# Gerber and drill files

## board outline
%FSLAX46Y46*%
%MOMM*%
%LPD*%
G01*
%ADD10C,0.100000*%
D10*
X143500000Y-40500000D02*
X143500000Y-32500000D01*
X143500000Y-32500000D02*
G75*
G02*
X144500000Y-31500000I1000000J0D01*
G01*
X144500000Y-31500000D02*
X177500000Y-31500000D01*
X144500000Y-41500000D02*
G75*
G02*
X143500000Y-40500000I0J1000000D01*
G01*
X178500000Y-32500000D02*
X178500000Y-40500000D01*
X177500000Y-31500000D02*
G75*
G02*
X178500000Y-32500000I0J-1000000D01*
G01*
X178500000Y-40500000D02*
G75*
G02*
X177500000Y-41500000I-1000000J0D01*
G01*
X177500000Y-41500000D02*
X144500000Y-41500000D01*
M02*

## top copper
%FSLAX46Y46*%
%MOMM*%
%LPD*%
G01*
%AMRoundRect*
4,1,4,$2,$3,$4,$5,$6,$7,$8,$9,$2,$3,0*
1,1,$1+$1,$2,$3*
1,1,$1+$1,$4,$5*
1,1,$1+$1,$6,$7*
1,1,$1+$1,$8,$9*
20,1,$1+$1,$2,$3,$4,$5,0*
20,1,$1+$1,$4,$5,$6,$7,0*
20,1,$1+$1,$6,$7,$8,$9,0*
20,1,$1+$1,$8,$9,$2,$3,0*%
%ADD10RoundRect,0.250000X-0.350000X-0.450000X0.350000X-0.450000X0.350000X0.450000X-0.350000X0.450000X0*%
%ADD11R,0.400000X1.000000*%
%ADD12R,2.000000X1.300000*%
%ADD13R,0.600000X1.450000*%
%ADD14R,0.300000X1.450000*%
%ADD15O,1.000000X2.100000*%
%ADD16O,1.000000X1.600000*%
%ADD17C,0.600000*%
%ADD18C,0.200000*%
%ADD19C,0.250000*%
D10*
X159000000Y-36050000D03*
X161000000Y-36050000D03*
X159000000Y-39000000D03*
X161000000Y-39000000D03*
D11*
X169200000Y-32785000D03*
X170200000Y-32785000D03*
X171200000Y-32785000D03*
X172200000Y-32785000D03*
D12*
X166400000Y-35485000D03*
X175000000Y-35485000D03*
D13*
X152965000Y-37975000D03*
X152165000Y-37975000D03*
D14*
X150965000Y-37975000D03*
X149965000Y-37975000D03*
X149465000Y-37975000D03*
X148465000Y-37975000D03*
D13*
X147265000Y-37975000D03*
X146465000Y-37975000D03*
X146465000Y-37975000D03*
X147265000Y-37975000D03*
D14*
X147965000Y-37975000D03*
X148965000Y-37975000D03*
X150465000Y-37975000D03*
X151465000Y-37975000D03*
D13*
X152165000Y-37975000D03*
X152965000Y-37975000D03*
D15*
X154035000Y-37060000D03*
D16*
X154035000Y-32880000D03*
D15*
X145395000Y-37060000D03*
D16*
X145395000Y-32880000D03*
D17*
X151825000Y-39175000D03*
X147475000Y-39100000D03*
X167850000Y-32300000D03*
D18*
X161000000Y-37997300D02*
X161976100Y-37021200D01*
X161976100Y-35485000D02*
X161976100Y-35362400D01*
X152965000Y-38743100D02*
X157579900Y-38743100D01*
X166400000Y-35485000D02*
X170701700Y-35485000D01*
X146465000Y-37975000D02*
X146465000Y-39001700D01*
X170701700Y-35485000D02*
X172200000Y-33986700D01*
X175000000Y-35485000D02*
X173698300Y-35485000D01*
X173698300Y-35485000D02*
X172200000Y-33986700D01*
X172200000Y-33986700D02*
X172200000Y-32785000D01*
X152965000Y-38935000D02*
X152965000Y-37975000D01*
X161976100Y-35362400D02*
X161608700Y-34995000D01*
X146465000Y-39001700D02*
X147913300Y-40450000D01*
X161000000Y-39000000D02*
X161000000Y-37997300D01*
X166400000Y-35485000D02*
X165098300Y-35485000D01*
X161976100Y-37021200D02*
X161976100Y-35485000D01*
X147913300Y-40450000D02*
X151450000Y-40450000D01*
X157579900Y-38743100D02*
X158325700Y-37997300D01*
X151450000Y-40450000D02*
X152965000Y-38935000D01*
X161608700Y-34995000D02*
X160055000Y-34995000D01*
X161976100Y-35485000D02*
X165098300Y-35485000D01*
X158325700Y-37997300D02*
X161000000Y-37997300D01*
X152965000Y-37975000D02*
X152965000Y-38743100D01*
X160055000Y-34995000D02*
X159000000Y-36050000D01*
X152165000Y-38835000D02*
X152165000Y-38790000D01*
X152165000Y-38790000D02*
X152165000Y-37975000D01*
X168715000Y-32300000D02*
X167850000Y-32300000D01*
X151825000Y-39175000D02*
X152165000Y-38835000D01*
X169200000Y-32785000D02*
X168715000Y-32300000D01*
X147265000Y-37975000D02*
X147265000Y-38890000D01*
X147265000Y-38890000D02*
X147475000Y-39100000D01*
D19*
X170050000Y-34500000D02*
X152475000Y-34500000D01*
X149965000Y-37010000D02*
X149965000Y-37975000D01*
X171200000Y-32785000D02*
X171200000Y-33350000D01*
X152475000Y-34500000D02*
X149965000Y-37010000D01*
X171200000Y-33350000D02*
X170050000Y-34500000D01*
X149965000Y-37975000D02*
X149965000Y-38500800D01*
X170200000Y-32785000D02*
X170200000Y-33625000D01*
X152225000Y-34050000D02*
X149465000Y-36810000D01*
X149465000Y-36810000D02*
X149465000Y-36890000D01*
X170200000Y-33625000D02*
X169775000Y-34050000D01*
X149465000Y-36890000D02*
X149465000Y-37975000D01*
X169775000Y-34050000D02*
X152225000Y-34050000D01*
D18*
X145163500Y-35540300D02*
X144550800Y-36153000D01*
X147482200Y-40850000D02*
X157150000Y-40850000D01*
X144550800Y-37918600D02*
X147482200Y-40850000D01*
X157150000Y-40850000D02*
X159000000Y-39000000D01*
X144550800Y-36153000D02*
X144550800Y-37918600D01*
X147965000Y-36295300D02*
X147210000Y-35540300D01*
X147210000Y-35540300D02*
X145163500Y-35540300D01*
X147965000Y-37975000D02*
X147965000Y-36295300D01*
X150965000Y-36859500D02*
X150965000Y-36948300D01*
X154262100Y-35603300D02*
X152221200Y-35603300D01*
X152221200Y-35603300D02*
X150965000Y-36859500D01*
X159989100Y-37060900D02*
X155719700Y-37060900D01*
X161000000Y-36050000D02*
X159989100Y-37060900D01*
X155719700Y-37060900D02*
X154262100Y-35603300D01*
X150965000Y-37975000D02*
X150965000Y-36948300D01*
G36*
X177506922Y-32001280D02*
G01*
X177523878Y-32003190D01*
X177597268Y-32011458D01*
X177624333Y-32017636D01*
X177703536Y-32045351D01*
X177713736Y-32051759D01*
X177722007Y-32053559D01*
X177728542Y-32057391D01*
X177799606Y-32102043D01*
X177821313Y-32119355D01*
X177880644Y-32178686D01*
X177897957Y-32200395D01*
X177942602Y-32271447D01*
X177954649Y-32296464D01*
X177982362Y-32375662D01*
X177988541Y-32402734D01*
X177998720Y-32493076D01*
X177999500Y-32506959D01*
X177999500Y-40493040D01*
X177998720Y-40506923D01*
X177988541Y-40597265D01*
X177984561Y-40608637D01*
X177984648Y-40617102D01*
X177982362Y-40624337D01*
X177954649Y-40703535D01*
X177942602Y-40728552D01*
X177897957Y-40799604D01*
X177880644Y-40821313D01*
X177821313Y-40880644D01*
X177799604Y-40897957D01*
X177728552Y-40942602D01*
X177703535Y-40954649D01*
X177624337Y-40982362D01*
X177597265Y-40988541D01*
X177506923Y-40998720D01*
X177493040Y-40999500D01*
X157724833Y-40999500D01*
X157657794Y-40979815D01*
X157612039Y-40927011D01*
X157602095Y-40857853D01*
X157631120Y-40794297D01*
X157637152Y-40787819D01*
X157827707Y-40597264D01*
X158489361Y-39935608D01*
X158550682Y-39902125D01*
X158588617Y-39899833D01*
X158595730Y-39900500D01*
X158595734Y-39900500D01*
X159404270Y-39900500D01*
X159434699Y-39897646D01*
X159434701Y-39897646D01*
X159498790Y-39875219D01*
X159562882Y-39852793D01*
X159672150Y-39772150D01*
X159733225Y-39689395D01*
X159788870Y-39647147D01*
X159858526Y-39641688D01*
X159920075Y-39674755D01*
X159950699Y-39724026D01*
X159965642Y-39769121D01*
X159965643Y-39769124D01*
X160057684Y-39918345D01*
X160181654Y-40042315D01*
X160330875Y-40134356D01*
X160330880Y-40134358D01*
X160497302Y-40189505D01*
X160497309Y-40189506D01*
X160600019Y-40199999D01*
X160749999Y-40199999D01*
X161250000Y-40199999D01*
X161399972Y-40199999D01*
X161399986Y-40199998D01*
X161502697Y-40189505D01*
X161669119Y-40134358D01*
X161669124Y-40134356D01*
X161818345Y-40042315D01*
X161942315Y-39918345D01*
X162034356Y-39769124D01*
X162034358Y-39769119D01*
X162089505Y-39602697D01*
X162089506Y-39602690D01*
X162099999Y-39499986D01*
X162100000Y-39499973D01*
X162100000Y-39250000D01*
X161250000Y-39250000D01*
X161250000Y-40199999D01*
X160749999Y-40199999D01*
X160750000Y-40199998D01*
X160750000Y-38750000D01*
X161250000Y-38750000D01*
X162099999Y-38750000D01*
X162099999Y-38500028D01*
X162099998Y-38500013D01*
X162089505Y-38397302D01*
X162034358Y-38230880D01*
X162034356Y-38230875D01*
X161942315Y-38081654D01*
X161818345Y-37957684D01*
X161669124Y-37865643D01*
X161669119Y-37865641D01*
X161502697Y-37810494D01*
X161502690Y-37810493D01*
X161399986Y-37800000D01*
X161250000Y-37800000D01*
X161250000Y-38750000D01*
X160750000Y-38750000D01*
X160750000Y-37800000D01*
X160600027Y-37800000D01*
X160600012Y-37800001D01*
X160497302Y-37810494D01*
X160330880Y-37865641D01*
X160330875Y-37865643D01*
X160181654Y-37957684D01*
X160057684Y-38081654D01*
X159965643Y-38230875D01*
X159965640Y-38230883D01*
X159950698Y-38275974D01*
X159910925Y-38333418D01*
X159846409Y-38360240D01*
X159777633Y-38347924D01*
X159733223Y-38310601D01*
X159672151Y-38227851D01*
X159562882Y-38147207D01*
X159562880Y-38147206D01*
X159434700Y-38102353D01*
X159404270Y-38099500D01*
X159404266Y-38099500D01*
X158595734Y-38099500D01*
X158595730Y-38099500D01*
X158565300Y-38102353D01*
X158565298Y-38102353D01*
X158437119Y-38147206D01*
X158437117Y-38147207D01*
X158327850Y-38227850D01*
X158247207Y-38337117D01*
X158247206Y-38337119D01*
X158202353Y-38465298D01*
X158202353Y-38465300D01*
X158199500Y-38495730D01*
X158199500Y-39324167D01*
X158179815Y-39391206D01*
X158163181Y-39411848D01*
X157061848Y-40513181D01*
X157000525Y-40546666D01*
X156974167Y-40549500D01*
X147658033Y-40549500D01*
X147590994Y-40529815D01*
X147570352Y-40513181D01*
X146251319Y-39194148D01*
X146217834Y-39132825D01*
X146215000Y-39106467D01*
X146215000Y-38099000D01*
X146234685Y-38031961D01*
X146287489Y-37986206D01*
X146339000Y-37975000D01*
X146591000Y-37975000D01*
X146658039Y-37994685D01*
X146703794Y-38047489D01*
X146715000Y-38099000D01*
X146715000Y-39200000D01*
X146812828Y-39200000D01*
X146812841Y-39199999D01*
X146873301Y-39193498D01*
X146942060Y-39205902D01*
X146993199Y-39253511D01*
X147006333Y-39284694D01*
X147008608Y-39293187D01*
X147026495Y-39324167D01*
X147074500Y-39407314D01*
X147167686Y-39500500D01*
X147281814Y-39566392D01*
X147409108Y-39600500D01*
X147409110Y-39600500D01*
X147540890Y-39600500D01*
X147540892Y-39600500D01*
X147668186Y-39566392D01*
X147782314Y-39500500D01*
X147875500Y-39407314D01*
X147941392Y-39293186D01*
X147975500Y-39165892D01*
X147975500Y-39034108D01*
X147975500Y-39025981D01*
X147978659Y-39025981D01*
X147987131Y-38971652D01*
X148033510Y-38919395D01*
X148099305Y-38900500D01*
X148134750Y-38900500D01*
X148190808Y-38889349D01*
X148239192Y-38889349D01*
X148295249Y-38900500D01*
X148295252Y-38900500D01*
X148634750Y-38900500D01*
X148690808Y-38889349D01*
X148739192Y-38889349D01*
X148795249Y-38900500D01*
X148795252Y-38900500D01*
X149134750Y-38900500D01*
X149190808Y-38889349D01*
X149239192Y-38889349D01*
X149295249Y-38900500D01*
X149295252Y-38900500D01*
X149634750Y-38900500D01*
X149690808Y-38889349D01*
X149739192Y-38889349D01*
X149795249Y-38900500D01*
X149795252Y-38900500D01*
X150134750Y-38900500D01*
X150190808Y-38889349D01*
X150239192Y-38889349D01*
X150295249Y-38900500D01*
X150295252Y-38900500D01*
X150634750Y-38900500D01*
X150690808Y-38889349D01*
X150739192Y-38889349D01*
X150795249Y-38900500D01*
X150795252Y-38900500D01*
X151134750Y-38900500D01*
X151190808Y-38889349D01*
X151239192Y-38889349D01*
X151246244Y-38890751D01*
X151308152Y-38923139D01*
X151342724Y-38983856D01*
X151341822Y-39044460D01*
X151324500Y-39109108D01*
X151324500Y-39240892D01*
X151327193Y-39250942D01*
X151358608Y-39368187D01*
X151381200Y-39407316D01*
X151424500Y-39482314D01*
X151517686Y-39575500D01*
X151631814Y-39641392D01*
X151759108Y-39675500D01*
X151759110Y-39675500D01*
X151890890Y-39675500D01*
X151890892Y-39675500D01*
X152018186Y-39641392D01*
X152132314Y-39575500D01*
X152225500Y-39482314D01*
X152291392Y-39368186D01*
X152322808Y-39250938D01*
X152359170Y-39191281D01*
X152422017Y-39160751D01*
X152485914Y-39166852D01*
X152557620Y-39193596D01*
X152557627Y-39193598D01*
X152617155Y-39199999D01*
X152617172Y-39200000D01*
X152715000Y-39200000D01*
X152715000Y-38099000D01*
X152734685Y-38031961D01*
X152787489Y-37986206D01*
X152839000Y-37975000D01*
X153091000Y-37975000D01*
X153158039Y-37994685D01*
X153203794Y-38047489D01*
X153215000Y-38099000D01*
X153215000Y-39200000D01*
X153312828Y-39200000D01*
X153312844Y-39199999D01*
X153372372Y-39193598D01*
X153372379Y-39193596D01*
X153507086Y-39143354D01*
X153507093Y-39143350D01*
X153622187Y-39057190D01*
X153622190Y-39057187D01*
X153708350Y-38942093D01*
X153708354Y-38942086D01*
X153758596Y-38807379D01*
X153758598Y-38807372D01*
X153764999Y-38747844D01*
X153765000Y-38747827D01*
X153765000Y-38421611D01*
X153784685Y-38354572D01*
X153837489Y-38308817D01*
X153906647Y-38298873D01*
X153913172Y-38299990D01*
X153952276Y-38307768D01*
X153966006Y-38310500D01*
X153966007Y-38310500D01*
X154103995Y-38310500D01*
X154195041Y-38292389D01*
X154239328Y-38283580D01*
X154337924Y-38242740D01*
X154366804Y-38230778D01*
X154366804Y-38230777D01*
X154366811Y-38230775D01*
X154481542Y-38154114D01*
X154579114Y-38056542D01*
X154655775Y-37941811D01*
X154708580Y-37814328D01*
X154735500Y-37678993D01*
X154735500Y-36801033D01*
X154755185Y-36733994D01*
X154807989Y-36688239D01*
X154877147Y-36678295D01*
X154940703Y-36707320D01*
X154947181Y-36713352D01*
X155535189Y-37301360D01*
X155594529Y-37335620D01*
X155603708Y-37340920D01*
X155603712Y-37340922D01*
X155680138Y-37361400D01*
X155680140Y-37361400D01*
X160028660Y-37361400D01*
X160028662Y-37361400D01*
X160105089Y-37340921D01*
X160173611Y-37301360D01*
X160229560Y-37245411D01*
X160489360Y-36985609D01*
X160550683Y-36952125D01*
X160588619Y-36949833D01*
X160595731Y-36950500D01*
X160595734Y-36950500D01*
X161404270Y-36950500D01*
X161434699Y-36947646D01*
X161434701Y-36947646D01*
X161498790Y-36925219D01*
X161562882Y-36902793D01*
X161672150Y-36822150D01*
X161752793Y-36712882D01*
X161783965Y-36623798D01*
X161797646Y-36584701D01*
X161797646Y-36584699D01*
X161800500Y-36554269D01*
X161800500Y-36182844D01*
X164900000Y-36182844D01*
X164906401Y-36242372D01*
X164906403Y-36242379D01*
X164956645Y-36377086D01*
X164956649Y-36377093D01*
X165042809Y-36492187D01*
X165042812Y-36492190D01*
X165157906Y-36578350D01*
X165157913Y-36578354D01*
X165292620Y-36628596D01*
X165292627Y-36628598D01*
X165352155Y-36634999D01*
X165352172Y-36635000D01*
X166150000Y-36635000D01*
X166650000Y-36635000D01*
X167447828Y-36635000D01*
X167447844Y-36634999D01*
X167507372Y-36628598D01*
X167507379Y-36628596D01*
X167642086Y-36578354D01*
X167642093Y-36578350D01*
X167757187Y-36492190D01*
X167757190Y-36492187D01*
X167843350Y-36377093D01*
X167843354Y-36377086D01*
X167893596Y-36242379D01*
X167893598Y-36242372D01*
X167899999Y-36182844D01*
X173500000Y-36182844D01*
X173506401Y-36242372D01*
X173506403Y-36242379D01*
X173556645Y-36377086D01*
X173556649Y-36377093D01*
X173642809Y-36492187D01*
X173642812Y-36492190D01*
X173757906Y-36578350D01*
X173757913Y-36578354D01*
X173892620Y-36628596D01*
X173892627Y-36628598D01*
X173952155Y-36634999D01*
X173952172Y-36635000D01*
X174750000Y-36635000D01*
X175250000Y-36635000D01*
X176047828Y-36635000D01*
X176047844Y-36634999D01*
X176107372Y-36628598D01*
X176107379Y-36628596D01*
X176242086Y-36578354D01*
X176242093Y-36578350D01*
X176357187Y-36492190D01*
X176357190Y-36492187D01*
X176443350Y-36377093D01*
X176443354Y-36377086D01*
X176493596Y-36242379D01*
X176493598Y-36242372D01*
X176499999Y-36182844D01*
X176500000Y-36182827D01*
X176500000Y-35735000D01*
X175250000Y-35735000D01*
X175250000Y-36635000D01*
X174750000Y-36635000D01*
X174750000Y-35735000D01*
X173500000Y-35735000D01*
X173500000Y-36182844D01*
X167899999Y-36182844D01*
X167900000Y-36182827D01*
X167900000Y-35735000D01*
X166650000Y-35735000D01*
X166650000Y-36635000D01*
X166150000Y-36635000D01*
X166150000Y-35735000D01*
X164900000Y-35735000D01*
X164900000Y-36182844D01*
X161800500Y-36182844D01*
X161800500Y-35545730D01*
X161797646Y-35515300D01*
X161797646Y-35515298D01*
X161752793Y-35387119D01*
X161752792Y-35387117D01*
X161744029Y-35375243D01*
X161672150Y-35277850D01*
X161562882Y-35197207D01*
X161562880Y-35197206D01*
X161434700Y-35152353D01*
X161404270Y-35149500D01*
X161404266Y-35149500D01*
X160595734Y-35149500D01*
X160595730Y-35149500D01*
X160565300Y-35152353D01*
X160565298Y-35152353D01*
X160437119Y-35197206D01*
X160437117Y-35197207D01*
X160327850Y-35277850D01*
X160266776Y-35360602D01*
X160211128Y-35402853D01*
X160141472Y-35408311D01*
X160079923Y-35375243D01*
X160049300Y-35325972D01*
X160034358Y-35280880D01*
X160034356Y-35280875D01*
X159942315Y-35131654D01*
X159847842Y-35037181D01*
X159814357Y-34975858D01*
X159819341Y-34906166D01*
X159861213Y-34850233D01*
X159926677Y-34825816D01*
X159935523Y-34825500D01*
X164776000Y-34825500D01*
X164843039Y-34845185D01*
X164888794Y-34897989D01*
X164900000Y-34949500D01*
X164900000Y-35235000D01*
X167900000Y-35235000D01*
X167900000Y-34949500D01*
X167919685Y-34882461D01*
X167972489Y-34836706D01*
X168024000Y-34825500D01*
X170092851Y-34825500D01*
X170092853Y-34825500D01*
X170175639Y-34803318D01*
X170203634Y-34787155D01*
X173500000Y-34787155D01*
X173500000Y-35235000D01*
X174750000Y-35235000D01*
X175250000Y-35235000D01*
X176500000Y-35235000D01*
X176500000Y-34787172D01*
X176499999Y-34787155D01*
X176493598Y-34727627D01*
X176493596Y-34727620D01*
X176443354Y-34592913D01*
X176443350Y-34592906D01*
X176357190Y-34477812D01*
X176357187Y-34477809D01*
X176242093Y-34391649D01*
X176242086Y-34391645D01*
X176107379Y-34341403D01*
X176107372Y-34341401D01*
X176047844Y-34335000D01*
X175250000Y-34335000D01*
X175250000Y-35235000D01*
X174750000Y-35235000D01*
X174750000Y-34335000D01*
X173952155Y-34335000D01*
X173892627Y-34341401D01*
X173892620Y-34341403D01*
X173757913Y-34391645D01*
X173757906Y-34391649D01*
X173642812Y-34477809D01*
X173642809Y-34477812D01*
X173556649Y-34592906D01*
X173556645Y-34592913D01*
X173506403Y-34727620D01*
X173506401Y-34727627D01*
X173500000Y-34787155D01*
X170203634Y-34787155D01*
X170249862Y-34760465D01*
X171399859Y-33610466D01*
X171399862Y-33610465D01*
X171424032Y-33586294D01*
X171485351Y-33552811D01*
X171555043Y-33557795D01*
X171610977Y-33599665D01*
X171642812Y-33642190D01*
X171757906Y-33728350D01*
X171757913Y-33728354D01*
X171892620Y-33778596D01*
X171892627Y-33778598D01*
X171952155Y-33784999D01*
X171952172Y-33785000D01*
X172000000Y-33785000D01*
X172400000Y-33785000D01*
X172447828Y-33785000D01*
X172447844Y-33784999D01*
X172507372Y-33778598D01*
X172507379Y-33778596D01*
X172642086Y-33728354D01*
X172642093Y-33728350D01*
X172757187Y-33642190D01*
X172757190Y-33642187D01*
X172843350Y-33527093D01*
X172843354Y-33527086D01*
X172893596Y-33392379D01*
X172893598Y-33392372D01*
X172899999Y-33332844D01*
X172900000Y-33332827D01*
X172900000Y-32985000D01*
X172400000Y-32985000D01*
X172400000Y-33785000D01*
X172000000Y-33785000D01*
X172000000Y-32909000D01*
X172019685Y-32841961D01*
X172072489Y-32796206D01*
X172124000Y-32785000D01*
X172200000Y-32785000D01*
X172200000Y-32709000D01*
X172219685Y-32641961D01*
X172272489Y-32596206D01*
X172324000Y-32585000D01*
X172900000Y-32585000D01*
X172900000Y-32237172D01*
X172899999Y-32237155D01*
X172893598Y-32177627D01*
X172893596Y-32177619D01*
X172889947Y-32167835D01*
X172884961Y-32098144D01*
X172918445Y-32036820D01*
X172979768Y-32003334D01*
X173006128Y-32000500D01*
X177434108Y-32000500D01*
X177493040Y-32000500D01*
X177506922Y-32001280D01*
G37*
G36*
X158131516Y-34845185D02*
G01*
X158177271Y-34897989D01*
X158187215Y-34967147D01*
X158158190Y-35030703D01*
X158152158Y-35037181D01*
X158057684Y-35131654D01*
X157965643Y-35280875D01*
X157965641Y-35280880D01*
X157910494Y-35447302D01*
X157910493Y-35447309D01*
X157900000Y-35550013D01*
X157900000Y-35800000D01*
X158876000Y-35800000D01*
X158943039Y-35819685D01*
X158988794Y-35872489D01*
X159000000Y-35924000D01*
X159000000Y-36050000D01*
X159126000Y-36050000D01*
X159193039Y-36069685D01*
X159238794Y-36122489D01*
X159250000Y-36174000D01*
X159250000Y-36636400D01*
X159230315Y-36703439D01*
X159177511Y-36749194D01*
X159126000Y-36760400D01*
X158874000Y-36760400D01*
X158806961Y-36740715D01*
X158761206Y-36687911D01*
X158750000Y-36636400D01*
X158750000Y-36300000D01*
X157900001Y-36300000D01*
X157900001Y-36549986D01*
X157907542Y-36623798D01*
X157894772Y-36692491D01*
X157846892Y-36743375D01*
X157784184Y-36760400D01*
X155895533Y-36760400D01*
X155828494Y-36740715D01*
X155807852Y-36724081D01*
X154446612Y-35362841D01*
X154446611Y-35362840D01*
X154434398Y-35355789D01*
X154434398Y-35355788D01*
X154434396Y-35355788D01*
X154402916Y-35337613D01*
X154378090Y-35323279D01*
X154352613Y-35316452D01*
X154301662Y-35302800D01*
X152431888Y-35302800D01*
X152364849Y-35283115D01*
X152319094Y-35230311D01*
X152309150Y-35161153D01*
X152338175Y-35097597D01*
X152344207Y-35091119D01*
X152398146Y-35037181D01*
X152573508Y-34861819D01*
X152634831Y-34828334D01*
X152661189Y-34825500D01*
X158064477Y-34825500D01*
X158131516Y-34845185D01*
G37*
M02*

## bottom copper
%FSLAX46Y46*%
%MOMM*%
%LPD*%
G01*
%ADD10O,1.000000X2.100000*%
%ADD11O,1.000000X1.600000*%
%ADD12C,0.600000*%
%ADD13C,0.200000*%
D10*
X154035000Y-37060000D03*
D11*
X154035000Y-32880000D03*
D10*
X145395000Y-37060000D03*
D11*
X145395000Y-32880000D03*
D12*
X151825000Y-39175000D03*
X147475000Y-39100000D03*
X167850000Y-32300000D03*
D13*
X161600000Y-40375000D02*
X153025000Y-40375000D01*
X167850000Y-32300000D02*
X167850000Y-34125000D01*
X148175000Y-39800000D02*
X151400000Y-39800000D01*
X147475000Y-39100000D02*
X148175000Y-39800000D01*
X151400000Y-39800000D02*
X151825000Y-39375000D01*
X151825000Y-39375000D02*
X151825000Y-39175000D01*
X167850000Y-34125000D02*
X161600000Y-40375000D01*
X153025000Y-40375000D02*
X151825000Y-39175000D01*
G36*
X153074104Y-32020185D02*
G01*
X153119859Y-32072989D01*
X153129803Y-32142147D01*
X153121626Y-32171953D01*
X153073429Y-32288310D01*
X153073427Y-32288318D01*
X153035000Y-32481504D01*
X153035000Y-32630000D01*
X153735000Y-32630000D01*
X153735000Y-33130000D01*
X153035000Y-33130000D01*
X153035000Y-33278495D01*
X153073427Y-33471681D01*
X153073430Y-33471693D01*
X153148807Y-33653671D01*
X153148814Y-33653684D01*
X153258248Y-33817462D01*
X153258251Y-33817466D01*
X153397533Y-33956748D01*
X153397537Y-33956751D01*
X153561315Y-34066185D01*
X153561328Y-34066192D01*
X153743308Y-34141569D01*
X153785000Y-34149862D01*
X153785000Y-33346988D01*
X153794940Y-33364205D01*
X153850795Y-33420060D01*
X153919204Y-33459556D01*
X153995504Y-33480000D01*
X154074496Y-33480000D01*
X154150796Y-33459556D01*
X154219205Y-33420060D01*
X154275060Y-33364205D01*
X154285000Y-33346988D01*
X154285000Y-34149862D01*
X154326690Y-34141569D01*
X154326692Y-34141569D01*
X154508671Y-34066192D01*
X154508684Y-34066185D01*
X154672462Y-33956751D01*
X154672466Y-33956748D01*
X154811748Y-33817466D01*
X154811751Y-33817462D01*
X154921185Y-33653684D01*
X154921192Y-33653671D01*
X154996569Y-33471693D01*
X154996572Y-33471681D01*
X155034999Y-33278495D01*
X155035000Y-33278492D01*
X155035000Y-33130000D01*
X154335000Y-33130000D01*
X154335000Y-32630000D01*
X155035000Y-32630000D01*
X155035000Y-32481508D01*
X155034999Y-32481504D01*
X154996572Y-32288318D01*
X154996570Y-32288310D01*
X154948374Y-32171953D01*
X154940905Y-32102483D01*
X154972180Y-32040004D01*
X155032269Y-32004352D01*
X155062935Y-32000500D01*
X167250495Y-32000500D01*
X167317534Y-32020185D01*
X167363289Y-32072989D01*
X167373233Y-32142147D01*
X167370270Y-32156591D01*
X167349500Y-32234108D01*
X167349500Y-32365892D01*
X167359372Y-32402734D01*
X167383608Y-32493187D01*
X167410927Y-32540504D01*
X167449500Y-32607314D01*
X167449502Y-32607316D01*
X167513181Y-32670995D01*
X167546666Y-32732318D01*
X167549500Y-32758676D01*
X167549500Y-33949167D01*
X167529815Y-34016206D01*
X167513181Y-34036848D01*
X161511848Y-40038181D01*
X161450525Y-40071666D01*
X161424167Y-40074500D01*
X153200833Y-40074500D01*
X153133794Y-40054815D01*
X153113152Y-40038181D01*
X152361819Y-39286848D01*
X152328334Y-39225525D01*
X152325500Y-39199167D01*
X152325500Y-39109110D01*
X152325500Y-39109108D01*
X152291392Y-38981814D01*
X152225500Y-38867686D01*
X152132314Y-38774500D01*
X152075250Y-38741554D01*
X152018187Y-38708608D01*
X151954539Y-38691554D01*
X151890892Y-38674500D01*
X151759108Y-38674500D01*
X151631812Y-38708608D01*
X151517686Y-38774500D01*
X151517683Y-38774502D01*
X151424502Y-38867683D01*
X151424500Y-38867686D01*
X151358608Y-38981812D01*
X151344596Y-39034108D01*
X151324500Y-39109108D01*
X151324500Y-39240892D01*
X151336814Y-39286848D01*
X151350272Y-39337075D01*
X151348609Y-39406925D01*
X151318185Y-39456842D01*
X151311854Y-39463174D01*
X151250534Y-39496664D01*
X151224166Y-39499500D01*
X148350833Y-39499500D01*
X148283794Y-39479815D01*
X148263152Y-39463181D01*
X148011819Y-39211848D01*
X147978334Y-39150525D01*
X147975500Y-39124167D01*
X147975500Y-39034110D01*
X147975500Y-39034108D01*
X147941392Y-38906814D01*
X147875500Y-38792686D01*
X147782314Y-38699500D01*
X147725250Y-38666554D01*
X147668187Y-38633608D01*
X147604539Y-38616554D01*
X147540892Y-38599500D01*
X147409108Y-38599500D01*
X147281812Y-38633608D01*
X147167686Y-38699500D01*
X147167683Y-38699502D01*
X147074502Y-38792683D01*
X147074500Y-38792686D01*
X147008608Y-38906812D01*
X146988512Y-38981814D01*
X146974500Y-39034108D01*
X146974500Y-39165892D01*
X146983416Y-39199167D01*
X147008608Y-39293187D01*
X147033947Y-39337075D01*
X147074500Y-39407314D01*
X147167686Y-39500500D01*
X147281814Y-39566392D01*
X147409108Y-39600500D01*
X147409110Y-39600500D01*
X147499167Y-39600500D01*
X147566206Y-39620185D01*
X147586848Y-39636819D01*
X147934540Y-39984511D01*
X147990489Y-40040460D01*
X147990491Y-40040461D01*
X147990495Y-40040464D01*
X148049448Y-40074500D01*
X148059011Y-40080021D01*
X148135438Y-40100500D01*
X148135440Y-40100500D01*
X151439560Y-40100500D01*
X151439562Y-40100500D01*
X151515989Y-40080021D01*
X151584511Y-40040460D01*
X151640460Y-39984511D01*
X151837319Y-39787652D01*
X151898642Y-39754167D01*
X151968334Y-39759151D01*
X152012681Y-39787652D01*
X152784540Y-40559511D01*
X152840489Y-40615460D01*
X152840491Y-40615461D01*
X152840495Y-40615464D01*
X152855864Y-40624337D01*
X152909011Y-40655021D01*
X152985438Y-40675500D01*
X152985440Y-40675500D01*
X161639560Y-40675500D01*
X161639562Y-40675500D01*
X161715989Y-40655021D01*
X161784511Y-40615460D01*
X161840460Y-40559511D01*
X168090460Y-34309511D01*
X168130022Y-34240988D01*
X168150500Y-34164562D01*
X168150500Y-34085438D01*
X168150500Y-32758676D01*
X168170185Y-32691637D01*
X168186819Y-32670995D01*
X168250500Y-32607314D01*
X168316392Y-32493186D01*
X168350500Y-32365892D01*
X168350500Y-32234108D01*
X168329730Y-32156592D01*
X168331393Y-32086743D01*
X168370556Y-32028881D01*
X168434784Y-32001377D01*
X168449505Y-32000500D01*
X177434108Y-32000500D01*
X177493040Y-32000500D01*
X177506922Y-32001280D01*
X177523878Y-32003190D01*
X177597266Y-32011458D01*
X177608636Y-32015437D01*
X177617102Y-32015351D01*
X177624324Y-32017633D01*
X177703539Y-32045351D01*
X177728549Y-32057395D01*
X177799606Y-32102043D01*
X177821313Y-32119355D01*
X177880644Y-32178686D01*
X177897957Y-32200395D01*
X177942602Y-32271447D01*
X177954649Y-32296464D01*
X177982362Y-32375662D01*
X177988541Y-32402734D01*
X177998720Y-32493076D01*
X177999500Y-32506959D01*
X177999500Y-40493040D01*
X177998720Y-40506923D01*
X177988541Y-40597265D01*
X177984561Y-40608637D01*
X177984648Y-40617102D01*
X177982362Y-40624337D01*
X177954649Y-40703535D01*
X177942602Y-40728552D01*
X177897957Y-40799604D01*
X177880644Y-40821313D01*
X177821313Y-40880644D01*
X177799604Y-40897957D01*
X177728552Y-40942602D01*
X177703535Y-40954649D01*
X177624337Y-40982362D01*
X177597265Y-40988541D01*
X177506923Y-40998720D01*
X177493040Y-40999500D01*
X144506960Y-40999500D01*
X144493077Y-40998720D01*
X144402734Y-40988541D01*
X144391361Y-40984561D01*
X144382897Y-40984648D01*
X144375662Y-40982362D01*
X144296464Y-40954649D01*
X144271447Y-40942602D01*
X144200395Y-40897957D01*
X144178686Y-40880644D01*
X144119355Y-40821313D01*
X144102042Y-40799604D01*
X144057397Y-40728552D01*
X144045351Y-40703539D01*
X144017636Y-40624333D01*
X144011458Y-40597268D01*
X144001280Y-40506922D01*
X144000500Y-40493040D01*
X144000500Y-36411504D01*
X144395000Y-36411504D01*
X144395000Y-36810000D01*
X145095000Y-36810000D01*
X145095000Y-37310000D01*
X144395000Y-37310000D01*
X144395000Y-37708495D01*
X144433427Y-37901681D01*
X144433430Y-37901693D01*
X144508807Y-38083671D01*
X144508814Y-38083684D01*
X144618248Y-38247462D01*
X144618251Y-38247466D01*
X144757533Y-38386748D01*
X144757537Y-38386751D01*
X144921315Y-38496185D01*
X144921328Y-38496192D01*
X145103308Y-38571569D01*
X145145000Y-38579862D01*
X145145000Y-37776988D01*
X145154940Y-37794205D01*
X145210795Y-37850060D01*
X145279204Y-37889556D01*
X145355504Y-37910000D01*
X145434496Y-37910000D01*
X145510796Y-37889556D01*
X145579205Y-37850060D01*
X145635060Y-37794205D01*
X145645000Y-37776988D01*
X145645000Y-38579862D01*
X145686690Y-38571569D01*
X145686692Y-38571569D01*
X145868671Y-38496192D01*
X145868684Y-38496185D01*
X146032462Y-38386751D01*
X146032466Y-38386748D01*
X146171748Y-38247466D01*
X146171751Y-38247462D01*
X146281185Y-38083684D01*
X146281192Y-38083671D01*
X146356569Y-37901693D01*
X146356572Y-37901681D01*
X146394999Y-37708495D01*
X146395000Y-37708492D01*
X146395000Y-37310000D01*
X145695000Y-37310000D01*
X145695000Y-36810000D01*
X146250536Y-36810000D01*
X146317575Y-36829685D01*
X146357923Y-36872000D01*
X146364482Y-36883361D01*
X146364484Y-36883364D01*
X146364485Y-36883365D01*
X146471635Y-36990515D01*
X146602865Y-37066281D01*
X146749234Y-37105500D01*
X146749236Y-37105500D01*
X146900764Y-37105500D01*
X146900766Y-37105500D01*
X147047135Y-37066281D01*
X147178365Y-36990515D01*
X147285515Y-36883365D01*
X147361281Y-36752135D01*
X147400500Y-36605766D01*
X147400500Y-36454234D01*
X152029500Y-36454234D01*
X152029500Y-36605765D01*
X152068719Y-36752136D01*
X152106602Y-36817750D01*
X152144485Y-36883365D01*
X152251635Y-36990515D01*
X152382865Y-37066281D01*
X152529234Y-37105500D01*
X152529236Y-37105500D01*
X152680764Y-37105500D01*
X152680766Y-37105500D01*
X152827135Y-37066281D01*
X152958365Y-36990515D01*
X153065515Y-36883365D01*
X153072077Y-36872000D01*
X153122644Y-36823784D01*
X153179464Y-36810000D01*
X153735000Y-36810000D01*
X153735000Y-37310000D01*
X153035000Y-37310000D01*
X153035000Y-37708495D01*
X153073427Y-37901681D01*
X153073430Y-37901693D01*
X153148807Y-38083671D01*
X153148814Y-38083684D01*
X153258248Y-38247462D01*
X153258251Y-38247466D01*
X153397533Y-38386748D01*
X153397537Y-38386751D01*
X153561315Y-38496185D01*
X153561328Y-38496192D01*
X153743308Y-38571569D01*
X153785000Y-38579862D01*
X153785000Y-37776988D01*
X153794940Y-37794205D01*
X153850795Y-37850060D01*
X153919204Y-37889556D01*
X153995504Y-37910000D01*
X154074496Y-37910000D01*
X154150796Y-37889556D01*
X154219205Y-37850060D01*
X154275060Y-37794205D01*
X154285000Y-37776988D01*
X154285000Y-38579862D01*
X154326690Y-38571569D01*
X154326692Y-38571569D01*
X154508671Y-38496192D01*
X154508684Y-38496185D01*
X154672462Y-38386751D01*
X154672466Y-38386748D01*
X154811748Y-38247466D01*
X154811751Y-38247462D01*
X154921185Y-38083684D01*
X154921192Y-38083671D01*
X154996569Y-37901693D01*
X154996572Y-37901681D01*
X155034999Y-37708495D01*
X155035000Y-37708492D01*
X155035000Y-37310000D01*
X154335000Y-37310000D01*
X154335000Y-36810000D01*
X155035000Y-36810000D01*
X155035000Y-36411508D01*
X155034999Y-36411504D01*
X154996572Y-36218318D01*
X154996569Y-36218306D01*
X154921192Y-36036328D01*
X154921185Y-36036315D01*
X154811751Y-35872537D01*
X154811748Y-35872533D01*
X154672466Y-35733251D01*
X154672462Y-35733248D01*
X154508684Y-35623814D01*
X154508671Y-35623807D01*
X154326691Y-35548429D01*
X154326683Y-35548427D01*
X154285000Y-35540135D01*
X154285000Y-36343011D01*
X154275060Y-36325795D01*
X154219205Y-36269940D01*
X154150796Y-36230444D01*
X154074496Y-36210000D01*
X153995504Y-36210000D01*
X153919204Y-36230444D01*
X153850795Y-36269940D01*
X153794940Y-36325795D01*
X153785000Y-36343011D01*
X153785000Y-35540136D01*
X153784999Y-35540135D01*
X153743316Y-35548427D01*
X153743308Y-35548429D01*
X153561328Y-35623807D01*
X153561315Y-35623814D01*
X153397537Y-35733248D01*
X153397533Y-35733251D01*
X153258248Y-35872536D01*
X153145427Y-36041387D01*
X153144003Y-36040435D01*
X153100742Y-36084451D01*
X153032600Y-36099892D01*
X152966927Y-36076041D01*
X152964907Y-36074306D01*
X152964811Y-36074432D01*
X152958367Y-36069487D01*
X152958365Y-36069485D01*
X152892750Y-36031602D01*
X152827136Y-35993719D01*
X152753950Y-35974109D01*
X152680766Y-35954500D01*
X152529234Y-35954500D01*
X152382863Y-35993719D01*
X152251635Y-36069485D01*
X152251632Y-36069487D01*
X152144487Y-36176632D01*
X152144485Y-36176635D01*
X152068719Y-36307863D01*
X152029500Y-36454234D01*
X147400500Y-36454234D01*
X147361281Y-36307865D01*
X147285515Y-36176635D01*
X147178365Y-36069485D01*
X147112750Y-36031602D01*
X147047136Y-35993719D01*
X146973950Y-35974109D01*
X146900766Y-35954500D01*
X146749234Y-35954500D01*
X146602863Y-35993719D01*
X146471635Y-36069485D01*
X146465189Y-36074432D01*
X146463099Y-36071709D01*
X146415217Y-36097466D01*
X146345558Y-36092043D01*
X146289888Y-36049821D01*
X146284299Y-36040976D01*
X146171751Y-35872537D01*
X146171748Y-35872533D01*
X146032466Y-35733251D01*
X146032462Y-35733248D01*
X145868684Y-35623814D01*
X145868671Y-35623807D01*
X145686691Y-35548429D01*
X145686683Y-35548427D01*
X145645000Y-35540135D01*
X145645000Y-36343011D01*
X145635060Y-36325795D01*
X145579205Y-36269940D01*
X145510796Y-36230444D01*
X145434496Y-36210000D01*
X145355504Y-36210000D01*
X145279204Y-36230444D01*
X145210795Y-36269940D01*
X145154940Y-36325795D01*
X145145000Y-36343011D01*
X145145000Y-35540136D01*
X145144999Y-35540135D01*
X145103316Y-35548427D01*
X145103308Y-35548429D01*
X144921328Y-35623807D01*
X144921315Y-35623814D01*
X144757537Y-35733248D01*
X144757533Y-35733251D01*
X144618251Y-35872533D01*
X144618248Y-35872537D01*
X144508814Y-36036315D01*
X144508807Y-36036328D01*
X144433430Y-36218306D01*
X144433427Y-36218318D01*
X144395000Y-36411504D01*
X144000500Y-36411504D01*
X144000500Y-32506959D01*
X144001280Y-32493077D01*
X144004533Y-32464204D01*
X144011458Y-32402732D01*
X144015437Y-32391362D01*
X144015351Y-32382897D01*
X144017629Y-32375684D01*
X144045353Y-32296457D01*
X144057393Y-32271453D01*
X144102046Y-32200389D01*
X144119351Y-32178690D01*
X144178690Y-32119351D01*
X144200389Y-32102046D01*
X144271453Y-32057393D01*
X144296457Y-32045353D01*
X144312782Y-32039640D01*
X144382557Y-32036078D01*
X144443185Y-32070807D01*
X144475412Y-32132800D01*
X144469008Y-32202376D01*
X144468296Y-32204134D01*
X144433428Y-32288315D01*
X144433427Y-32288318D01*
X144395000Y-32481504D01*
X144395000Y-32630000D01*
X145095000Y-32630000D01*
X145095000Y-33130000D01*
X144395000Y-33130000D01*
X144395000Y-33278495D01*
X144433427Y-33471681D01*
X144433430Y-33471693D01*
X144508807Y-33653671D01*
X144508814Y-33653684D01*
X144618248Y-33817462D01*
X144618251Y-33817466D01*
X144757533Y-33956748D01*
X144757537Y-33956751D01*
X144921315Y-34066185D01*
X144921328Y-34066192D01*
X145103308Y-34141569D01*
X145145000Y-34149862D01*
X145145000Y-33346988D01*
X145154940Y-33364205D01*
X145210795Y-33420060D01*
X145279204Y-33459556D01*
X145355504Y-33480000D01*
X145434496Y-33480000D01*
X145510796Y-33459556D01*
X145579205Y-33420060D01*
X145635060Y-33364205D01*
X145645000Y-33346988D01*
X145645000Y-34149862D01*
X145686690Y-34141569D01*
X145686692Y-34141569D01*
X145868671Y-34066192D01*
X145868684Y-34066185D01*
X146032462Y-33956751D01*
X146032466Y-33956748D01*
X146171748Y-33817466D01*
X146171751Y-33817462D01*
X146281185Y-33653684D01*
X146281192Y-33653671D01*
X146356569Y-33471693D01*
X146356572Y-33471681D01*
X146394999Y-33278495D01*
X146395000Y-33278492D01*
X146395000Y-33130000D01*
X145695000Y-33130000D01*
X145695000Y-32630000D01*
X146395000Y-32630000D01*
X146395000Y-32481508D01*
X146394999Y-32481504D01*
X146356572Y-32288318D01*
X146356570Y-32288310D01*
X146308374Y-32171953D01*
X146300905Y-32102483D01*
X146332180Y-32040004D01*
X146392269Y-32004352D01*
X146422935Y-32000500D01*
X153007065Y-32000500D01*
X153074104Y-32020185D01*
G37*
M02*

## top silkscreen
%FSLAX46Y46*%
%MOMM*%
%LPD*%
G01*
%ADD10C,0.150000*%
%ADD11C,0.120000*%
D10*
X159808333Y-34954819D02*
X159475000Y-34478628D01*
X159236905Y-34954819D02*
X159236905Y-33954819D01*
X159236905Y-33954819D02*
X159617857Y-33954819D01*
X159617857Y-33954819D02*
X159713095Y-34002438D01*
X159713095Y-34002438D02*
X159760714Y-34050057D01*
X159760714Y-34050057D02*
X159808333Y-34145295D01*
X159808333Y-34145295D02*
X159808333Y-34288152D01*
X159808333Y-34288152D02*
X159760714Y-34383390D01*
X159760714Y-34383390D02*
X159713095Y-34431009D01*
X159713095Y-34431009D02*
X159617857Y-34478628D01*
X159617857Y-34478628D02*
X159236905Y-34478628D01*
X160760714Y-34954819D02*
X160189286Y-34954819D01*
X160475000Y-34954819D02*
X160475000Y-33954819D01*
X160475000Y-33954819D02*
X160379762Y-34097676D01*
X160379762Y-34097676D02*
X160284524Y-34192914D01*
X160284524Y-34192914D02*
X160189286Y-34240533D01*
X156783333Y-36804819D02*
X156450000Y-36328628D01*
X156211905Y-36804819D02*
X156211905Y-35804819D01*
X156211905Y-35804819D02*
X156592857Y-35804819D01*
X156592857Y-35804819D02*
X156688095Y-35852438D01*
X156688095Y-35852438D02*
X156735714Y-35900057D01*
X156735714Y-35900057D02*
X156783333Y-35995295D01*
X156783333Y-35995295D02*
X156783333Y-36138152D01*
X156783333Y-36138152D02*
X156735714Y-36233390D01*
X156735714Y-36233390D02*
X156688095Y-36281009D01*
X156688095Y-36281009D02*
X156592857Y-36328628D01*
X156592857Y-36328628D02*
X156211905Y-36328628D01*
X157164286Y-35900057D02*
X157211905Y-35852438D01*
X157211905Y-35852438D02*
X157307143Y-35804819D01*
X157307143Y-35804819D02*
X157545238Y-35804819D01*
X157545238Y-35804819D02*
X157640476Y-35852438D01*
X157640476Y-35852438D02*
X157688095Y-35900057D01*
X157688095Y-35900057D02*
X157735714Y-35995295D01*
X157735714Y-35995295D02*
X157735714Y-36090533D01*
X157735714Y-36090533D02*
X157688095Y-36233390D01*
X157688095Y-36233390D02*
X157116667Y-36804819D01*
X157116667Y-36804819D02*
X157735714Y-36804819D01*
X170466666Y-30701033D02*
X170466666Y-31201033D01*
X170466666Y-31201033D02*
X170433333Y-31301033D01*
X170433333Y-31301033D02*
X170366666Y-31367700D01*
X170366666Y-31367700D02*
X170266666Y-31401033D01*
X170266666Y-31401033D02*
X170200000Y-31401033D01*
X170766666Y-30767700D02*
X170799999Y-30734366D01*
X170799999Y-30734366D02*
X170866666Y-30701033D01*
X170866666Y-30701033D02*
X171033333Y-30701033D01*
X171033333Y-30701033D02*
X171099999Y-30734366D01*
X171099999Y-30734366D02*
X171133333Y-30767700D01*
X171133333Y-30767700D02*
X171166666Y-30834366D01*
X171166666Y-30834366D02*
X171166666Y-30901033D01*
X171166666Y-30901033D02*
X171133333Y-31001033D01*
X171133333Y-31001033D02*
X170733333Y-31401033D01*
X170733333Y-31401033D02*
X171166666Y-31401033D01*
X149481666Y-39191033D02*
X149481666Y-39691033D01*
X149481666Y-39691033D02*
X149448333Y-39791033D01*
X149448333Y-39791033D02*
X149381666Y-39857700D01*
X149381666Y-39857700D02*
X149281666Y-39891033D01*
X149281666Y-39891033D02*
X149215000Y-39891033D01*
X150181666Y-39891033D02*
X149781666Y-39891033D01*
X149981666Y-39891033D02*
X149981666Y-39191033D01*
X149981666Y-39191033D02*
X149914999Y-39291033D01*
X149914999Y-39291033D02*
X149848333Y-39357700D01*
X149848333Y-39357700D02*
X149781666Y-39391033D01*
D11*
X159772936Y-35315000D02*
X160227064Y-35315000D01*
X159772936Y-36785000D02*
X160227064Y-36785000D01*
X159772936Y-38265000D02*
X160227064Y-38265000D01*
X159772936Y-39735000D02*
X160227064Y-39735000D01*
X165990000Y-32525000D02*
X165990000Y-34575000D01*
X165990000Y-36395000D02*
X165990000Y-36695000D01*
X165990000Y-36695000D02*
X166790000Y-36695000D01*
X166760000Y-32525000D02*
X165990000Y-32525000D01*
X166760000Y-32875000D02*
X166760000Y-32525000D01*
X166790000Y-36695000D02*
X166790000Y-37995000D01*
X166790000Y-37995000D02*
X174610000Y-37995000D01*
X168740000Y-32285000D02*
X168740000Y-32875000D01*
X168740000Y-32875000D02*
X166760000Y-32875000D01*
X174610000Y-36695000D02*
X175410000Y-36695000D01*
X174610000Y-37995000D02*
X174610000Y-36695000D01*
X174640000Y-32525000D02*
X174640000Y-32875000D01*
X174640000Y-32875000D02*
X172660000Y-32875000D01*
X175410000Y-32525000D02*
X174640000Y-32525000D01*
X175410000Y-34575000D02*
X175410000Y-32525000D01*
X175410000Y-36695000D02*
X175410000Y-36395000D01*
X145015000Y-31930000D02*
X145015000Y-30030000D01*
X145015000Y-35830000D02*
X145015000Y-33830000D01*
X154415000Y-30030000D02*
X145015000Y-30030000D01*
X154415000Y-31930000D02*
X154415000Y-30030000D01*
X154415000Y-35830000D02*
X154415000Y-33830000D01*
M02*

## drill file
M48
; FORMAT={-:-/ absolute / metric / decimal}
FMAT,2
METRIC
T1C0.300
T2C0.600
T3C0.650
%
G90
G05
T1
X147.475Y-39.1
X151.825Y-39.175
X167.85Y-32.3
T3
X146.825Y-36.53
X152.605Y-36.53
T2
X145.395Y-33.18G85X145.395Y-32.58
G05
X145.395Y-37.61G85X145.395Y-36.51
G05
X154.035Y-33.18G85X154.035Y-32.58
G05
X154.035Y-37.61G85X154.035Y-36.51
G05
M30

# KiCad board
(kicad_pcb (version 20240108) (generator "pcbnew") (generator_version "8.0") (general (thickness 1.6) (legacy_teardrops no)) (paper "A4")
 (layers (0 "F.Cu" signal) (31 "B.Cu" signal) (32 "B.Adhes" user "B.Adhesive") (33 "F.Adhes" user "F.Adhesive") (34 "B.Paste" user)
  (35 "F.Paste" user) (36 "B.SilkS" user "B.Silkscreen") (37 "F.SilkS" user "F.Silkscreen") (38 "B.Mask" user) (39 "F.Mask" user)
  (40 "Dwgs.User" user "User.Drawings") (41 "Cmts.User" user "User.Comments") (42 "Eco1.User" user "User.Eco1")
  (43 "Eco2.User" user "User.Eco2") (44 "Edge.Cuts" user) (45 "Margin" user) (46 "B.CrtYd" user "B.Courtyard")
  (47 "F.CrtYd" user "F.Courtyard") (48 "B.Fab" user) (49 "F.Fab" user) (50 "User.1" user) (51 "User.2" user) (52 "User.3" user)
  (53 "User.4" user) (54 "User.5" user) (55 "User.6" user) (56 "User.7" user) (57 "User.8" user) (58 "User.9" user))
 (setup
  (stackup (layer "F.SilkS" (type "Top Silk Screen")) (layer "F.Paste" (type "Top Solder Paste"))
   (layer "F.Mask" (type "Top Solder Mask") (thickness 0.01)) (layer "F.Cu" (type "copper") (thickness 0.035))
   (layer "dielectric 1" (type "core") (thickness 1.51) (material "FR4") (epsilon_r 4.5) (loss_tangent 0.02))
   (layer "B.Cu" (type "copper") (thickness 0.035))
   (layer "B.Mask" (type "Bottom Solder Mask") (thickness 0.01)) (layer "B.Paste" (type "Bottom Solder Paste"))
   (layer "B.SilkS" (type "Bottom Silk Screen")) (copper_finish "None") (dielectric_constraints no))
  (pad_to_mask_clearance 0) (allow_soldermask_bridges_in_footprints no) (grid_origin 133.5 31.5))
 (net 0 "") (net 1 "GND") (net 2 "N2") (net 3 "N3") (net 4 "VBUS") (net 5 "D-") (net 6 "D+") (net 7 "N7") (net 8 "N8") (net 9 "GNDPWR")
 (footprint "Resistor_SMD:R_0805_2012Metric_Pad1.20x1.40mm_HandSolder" (layer "F.Cu") (at 160 36.05)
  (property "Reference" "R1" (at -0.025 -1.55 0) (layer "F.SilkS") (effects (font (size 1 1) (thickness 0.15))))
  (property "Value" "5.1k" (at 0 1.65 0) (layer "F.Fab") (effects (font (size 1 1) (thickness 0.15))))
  (fp_line (start -0.227064 -0.735) (end 0.227064 -0.735) (stroke (width 0.12) (type solid)) (layer "F.SilkS"))
  (fp_line (start -0.227064 0.735) (end 0.227064 0.735) (stroke (width 0.12) (type solid)) (layer "F.SilkS"))
  (pad "1" smd roundrect (at -1 0) (size 1.2 1.4) (layers "F.Cu" "F.Paste" "F.Mask") (roundrect_rratio 0.208333) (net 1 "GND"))
  (pad "2" smd roundrect (at 1 0) (size 1.2 1.4) (layers "F.Cu" "F.Paste" "F.Mask") (roundrect_rratio 0.208333) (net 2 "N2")))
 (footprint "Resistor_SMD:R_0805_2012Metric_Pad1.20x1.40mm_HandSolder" (layer "F.Cu") (at 160 39)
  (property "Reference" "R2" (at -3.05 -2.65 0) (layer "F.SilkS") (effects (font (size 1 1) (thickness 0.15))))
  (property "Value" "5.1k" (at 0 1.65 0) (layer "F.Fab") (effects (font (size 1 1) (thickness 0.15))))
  (fp_line (start -0.227064 -0.735) (end 0.227064 -0.735) (stroke (width 0.12) (type solid)) (layer "F.SilkS"))
  (fp_line (start -0.227064 0.735) (end 0.227064 0.735) (stroke (width 0.12) (type solid)) (layer "F.SilkS"))
  (pad "1" smd roundrect (at -1 0) (size 1.2 1.4) (layers "F.Cu" "F.Paste" "F.Mask") (roundrect_rratio 0.208333) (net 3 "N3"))
  (pad "2" smd roundrect (at 1 0) (size 1.2 1.4) (layers "F.Cu" "F.Paste" "F.Mask") (roundrect_rratio 0.208333) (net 1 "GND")))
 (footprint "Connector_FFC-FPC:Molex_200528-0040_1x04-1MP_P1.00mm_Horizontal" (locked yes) (layer "F.Cu") (at 170.7 33.695)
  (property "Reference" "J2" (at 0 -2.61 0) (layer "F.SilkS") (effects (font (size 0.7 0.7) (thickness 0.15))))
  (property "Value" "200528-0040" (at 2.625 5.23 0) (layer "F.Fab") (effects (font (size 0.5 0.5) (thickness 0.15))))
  (fp_line (start -4.71 -1.17) (end -4.71 0.88) (stroke (width 0.12) (type solid)) (layer "F.SilkS"))
  (fp_line (start -4.71 2.7) (end -4.71 3) (stroke (width 0.12) (type solid)) (layer "F.SilkS"))
  (fp_line (start -4.71 3) (end -3.91 3) (stroke (width 0.12) (type solid)) (layer "F.SilkS"))
  (fp_line (start -3.94 -1.17) (end -4.71 -1.17) (stroke (width 0.12) (type solid)) (layer "F.SilkS"))
  (fp_line (start -3.94 -0.82) (end -3.94 -1.17) (stroke (width 0.12) (type solid)) (layer "F.SilkS"))
  (fp_line (start -3.91 3) (end -3.91 4.3) (stroke (width 0.12) (type solid)) (layer "F.SilkS"))
  (fp_line (start -3.91 4.3) (end 3.91 4.3) (stroke (width 0.12) (type solid)) (layer "F.SilkS"))
  (fp_line (start -1.96 -1.41) (end -1.96 -0.82) (stroke (width 0.12) (type solid)) (layer "F.SilkS"))
  (fp_line (start -1.96 -0.82) (end -3.94 -0.82) (stroke (width 0.12) (type solid)) (layer "F.SilkS"))
  (fp_line (start 3.91 3) (end 4.71 3) (stroke (width 0.12) (type solid)) (layer "F.SilkS"))
  (fp_line (start 3.91 4.3) (end 3.91 3) (stroke (width 0.12) (type solid)) (layer "F.SilkS"))
  (fp_line (start 3.94 -1.17) (end 3.94 -0.82) (stroke (width 0.12) (type solid)) (layer "F.SilkS"))
  (fp_line (start 3.94 -0.82) (end 1.96 -0.82) (stroke (width 0.12) (type solid)) (layer "F.SilkS"))
  (fp_line (start 4.71 -1.17) (end 3.94 -1.17) (stroke (width 0.12) (type solid)) (layer "F.SilkS"))
  (fp_line (start 4.71 0.88) (end 4.71 -1.17) (stroke (width 0.12) (type solid)) (layer "F.SilkS"))
  (fp_line (start 4.71 3) (end 4.71 2.7) (stroke (width 0.12) (type solid)) (layer "F.SilkS"))
  (pad "1" smd rect (at -1.5 -0.91) (size 0.4 1) (layers "F.Cu" "F.Paste" "F.Mask") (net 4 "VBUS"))
  (pad "2" smd rect (at -0.5 -0.91) (size 0.4 1) (layers "F.Cu" "F.Paste" "F.Mask") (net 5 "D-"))
  (pad "3" smd rect (at 0.5 -0.91) (size 0.4 1) (layers "F.Cu" "F.Paste" "F.Mask") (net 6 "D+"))
  (pad "4" smd rect (at 1.5 -0.91) (size 0.4 1) (layers "F.Cu" "F.Paste" "F.Mask") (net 1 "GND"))
  (pad "MP" smd rect (at -4.3 1.79) (size 2 1.3) (layers "F.Cu" "F.Paste" "F.Mask") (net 1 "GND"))
  (pad "MP" smd rect (at 4.3 1.79) (size 2 1.3) (layers "F.Cu" "F.Paste" "F.Mask") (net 1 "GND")))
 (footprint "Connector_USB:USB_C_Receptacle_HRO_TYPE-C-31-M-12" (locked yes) (layer "F.Cu") (at 149.715 33.93 180)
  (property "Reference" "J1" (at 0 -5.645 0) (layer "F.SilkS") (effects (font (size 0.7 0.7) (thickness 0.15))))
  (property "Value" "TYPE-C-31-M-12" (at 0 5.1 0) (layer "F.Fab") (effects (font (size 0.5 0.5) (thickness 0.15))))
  (fp_line (start 4.7 2) (end 4.7 3.9) (stroke (width 0.12) (type solid)) (layer "F.SilkS"))
  (fp_line (start 4.7 -1.9) (end 4.7 0.1) (stroke (width 0.12) (type solid)) (layer "F.SilkS"))
  (fp_line (start -4.7 3.9) (end 4.7 3.9) (stroke (width 0.12) (type solid)) (layer "F.SilkS"))
  (fp_line (start -4.7 2) (end -4.7 3.9) (stroke (width 0.12) (type solid)) (layer "F.SilkS"))
  (fp_line (start -4.7 -1.9) (end -4.7 0.1) (stroke (width 0.12) (type solid)) (layer "F.SilkS"))
  (pad "" np_thru_hole circle (at -2.89 -2.6 180) (size 0.65 0.65) (drill 0.65) (layers "*.Cu" "*.Mask"))
  (pad "" np_thru_hole circle (at 2.89 -2.6 180) (size 0.65 0.65) (drill 0.65) (layers "*.Cu" "*.Mask"))
  (pad "A1" smd rect (at -3.25 -4.045 180) (size 0.6 1.45) (layers "F.Cu" "F.Paste" "F.Mask") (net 1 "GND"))
  (pad "A4" smd rect (at -2.45 -4.045 180) (size 0.6 1.45) (layers "F.Cu" "F.Paste" "F.Mask") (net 4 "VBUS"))
  (pad "A5" smd rect (at -1.25 -4.045 180) (size 0.3 1.45) (layers "F.Cu" "F.Paste" "F.Mask") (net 2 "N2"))
  (pad "A6" smd rect (at -0.25 -4.045 180) (size 0.3 1.45) (layers "F.Cu" "F.Paste" "F.Mask") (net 6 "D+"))
  (pad "A7" smd rect (at 0.25 -4.045 180) (size 0.3 1.45) (layers "F.Cu" "F.Paste" "F.Mask") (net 5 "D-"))
  (pad "A8" smd rect (at 1.25 -4.045 180) (size 0.3 1.45) (layers "F.Cu" "F.Paste" "F.Mask") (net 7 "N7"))
  (pad "A9" smd rect (at 2.45 -4.045 180) (size 0.6 1.45) (layers "F.Cu" "F.Paste" "F.Mask") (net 4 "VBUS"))
  (pad "A12" smd rect (at 3.25 -4.045 180) (size 0.6 1.45) (layers "F.Cu" "F.Paste" "F.Mask") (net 1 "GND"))
  (pad "B1" smd rect (at 3.25 -4.045 180) (size 0.6 1.45) (layers "F.Cu" "F.Paste" "F.Mask") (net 1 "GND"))
  (pad "B4" smd rect (at 2.45 -4.045 180) (size 0.6 1.45) (layers "F.Cu" "F.Paste" "F.Mask") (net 4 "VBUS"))
  (pad "B5" smd rect (at 1.75 -4.045 180) (size 0.3 1.45) (layers "F.Cu" "F.Paste" "F.Mask") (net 3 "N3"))
  (pad "B6" smd rect (at 0.75 -4.045 180) (size 0.3 1.45) (layers "F.Cu" "F.Paste" "F.Mask") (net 6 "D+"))
  (pad "B7" smd rect (at -0.75 -4.045 180) (size 0.3 1.45) (layers "F.Cu" "F.Paste" "F.Mask") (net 5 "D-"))
  (pad "B8" smd rect (at -1.75 -4.045 180) (size 0.3 1.45) (layers "F.Cu" "F.Paste" "F.Mask") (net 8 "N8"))
  (pad "B9" smd rect (at -2.45 -4.045 180) (size 0.6 1.45) (layers "F.Cu" "F.Paste" "F.Mask") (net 4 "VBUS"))
  (pad "B12" smd rect (at -3.25 -4.045 180) (size 0.6 1.45) (layers "F.Cu" "F.Paste" "F.Mask") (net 1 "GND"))
  (pad "S1" thru_hole oval (at -4.32 -3.13 180) (size 1 2.1) (drill oval 0.6 1.7) (layers "*.Cu" "*.Mask") (remove_unused_layers no)
   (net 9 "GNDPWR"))
  (pad "S1" thru_hole oval (at -4.32 1.05 180) (size 1 1.6) (drill oval 0.6 1.2) (layers "*.Cu" "*.Mask") (remove_unused_layers no)
   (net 9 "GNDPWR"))
  (pad "S1" thru_hole oval (at 4.32 -3.13 180) (size 1 2.1) (drill oval 0.6 1.7) (layers "*.Cu" "*.Mask") (remove_unused_layers no)
   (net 9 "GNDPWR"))
  (pad "S1" thru_hole oval (at 4.32 1.05 180) (size 1 1.6) (drill oval 0.6 1.2) (layers "*.Cu" "*.Mask") (remove_unused_layers no)
   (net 9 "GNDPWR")))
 (gr_line (start 143.5 40.5) (end 143.5 32.5) (stroke (width 0.1) (type default)) (layer "Edge.Cuts"))
 (gr_arc (start 143.5 32.5) (mid 143.792893 31.792893) (end 144.5 31.5) (stroke (width 0.1) (type default)) (layer "Edge.Cuts"))
 (gr_line (start 144.5 31.5) (end 177.5 31.5) (stroke (width 0.1) (type default)) (layer "Edge.Cuts"))
 (gr_arc (start 144.5 41.5) (mid 143.792893 41.207107) (end 143.5 40.5) (stroke (width 0.1) (type default)) (layer "Edge.Cuts"))
 (gr_line (start 178.5 32.5) (end 178.5 40.5) (stroke (width 0.1) (type default)) (layer "Edge.Cuts"))
 (gr_arc (start 177.5 31.5) (mid 178.207107 31.792893) (end 178.5 32.5) (stroke (width 0.1) (type default)) (layer "Edge.Cuts"))
 (gr_arc (start 178.5 40.5) (mid 178.207107 41.207107) (end 177.5 41.5) (stroke (width 0.1) (type default)) (layer "Edge.Cuts"))
 (gr_line (start 177.5 41.5) (end 144.5 41.5) (stroke (width 0.1) (type default)) (layer "Edge.Cuts"))
 (segment (start 161 37.9973) (end 161.9761 37.0212) (width 0.2) (layer "F.Cu") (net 1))
 (segment (start 161.9761 35.485) (end 161.9761 35.3624) (width 0.2) (layer "F.Cu") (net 1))
 (segment (start 152.965 38.7431) (end 157.5799 38.7431) (width 0.2) (layer "F.Cu") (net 1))
 (segment (start 166.4 35.485) (end 170.7017 35.485) (width 0.2) (layer "F.Cu") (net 1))
 (segment (start 146.465 37.975) (end 146.465 39.0017) (width 0.2) (layer "F.Cu") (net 1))
 (segment (start 170.7017 35.485) (end 172.2 33.9867) (width 0.2) (layer "F.Cu") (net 1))
 (segment (start 175 35.485) (end 173.6983 35.485) (width 0.2) (layer "F.Cu") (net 1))
 (segment (start 173.6983 35.485) (end 172.2 33.9867) (width 0.2) (layer "F.Cu") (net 1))
 (segment (start 172.2 33.9867) (end 172.2 32.785) (width 0.2) (layer "F.Cu") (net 1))
 (segment (start 152.965 38.935) (end 152.965 37.975) (width 0.2) (layer "F.Cu") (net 1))
 (segment (start 161.9761 35.3624) (end 161.6087 34.995) (width 0.2) (layer "F.Cu") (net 1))
 (segment (start 146.465 39.0017) (end 147.9133 40.45) (width 0.2) (layer "F.Cu") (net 1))
 (segment (start 161 39) (end 161 37.9973) (width 0.2) (layer "F.Cu") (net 1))
 (segment (start 166.4 35.485) (end 165.0983 35.485) (width 0.2) (layer "F.Cu") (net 1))
 (segment (start 161.9761 37.0212) (end 161.9761 35.485) (width 0.2) (layer "F.Cu") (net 1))
 (segment (start 147.9133 40.45) (end 151.45 40.45) (width 0.2) (layer "F.Cu") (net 1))
 (segment (start 157.5799 38.7431) (end 158.3257 37.9973) (width 0.2) (layer "F.Cu") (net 1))
 (segment (start 151.45 40.45) (end 152.965 38.935) (width 0.2) (layer "F.Cu") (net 1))
 (segment (start 161.6087 34.995) (end 160.055 34.995) (width 0.2) (layer "F.Cu") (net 1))
 (segment (start 161.9761 35.485) (end 165.0983 35.485) (width 0.2) (layer "F.Cu") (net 1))
 (segment (start 158.3257 37.9973) (end 161 37.9973) (width 0.2) (layer "F.Cu") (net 1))
 (segment (start 152.965 37.975) (end 152.965 38.7431) (width 0.2) (layer "F.Cu") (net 1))
 (segment (start 160.055 34.995) (end 159 36.05) (width 0.2) (layer "F.Cu") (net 1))
 (segment (start 152.165 38.835) (end 152.165 38.79) (width 0.2) (layer "F.Cu") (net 4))
 (segment (start 152.165 38.79) (end 152.165 37.975) (width 0.2) (layer "F.Cu") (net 4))
 (segment (start 168.715 32.3) (end 167.85 32.3) (width 0.2) (layer "F.Cu") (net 4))
 (segment (start 151.825 39.175) (end 152.165 38.835) (width 0.2) (layer "F.Cu") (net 4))
 (segment (start 169.2 32.785) (end 168.715 32.3) (width 0.2) (layer "F.Cu") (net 4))
 (segment (start 147.265 37.975) (end 147.265 38.89) (width 0.2) (layer "F.Cu") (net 4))
 (segment (start 147.265 38.89) (end 147.475 39.1) (width 0.2) (layer "F.Cu") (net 4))
 (via (at 151.825 39.175) (size 0.6) (drill 0.3) (layers "F.Cu" "B.Cu") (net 4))
 (via (at 147.475 39.1) (size 0.6) (drill 0.3) (layers "F.Cu" "B.Cu") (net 4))
 (via (at 167.85 32.3) (size 0.6) (drill 0.3) (layers "F.Cu" "B.Cu") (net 4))
 (segment (start 161.6 40.375) (end 153.025 40.375) (width 0.2) (layer "B.Cu") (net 4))
 (segment (start 167.85 32.3) (end 167.85 34.125) (width 0.2) (layer "B.Cu") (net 4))
 (segment (start 148.175 39.8) (end 151.4 39.8) (width 0.2) (layer "B.Cu") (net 4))
 (segment (start 147.475 39.1) (end 148.175 39.8) (width 0.2) (layer "B.Cu") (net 4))
 (segment (start 151.4 39.8) (end 151.825 39.375) (width 0.2) (layer "B.Cu") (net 4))
 (segment (start 151.825 39.375) (end 151.825 39.175) (width 0.2) (layer "B.Cu") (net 4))
 (segment (start 167.85 34.125) (end 161.6 40.375) (width 0.2) (layer "B.Cu") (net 4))
 (segment (start 153.025 40.375) (end 151.825 39.175) (width 0.2) (layer "B.Cu") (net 4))
 (segment (start 170.05 34.5) (end 152.475 34.5) (width 0.25) (layer "F.Cu") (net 6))
 (segment (start 149.965 37.01) (end 149.965 37.975) (width 0.25) (layer "F.Cu") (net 6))
 (segment (start 171.2 32.785) (end 171.2 33.35) (width 0.25) (layer "F.Cu") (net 6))
 (segment (start 152.475 34.5) (end 149.965 37.01) (width 0.25) (layer "F.Cu") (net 6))
 (segment (start 171.2 33.35) (end 170.05 34.5) (width 0.25) (layer "F.Cu") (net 6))
 (segment (start 149.965 37.975) (end 149.965 38.5008) (width 0.25) (layer "F.Cu") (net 6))
 (segment (start 170.2 32.785) (end 170.2 33.625) (width 0.25) (layer "F.Cu") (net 5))
 (segment (start 152.225 34.05) (end 149.465 36.81) (width 0.25) (layer "F.Cu") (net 5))
 (segment (start 149.465 36.81) (end 149.465 36.89) (width 0.25) (layer "F.Cu") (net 5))
 (segment (start 170.2 33.625) (end 169.775 34.05) (width 0.25) (layer "F.Cu") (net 5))
 (segment (start 149.465 36.89) (end 149.465 37.975) (width 0.25) (layer "F.Cu") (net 5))
 (segment (start 169.775 34.05) (end 152.225 34.05) (width 0.25) (layer "F.Cu") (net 5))
 (segment (start 145.1635 35.5403) (end 144.5508 36.153) (width 0.2) (layer "F.Cu") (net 3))
 (segment (start 147.4822 40.85) (end 157.15 40.85) (width 0.2) (layer "F.Cu") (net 3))
 (segment (start 144.5508 37.9186) (end 147.4822 40.85) (width 0.2) (layer "F.Cu") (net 3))
 (segment (start 157.15 40.85) (end 159 39) (width 0.2) (layer "F.Cu") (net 3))
 (segment (start 144.5508 36.153) (end 144.5508 37.9186) (width 0.2) (layer "F.Cu") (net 3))
 (segment (start 147.965 36.2953) (end 147.21 35.5403) (width 0.2) (layer "F.Cu") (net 3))
 (segment (start 147.21 35.5403) (end 145.1635 35.5403) (width 0.2) (layer "F.Cu") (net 3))
 (segment (start 147.965 37.975) (end 147.965 36.2953) (width 0.2) (layer "F.Cu") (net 3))
 (segment (start 150.965 36.8595) (end 150.965 36.9483) (width 0.2) (layer "F.Cu") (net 2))
 (segment (start 154.2621 35.6033) (end 152.2212 35.6033) (width 0.2) (layer "F.Cu") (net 2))
 (segment (start 152.2212 35.6033) (end 150.965 36.8595) (width 0.2) (layer "F.Cu") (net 2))
 (segment (start 159.9891 37.0609) (end 155.7197 37.0609) (width 0.2) (layer "F.Cu") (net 2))
 (segment (start 161 36.05) (end 159.9891 37.0609) (width 0.2) (layer "F.Cu") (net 2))
 (segment (start 155.7197 37.0609) (end 154.2621 35.6033) (width 0.2) (layer "F.Cu") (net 2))
 (segment (start 150.965 37.975) (end 150.965 36.9483) (width 0.2) (layer "F.Cu") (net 2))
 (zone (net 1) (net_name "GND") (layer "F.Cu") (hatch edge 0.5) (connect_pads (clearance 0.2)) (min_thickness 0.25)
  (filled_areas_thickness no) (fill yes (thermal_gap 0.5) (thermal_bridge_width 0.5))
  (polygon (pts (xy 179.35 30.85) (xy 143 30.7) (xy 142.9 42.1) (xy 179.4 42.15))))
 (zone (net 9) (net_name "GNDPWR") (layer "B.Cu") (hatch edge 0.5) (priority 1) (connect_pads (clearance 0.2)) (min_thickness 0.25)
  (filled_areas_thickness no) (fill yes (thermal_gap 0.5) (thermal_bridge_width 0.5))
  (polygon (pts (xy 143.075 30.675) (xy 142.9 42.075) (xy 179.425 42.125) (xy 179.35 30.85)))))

